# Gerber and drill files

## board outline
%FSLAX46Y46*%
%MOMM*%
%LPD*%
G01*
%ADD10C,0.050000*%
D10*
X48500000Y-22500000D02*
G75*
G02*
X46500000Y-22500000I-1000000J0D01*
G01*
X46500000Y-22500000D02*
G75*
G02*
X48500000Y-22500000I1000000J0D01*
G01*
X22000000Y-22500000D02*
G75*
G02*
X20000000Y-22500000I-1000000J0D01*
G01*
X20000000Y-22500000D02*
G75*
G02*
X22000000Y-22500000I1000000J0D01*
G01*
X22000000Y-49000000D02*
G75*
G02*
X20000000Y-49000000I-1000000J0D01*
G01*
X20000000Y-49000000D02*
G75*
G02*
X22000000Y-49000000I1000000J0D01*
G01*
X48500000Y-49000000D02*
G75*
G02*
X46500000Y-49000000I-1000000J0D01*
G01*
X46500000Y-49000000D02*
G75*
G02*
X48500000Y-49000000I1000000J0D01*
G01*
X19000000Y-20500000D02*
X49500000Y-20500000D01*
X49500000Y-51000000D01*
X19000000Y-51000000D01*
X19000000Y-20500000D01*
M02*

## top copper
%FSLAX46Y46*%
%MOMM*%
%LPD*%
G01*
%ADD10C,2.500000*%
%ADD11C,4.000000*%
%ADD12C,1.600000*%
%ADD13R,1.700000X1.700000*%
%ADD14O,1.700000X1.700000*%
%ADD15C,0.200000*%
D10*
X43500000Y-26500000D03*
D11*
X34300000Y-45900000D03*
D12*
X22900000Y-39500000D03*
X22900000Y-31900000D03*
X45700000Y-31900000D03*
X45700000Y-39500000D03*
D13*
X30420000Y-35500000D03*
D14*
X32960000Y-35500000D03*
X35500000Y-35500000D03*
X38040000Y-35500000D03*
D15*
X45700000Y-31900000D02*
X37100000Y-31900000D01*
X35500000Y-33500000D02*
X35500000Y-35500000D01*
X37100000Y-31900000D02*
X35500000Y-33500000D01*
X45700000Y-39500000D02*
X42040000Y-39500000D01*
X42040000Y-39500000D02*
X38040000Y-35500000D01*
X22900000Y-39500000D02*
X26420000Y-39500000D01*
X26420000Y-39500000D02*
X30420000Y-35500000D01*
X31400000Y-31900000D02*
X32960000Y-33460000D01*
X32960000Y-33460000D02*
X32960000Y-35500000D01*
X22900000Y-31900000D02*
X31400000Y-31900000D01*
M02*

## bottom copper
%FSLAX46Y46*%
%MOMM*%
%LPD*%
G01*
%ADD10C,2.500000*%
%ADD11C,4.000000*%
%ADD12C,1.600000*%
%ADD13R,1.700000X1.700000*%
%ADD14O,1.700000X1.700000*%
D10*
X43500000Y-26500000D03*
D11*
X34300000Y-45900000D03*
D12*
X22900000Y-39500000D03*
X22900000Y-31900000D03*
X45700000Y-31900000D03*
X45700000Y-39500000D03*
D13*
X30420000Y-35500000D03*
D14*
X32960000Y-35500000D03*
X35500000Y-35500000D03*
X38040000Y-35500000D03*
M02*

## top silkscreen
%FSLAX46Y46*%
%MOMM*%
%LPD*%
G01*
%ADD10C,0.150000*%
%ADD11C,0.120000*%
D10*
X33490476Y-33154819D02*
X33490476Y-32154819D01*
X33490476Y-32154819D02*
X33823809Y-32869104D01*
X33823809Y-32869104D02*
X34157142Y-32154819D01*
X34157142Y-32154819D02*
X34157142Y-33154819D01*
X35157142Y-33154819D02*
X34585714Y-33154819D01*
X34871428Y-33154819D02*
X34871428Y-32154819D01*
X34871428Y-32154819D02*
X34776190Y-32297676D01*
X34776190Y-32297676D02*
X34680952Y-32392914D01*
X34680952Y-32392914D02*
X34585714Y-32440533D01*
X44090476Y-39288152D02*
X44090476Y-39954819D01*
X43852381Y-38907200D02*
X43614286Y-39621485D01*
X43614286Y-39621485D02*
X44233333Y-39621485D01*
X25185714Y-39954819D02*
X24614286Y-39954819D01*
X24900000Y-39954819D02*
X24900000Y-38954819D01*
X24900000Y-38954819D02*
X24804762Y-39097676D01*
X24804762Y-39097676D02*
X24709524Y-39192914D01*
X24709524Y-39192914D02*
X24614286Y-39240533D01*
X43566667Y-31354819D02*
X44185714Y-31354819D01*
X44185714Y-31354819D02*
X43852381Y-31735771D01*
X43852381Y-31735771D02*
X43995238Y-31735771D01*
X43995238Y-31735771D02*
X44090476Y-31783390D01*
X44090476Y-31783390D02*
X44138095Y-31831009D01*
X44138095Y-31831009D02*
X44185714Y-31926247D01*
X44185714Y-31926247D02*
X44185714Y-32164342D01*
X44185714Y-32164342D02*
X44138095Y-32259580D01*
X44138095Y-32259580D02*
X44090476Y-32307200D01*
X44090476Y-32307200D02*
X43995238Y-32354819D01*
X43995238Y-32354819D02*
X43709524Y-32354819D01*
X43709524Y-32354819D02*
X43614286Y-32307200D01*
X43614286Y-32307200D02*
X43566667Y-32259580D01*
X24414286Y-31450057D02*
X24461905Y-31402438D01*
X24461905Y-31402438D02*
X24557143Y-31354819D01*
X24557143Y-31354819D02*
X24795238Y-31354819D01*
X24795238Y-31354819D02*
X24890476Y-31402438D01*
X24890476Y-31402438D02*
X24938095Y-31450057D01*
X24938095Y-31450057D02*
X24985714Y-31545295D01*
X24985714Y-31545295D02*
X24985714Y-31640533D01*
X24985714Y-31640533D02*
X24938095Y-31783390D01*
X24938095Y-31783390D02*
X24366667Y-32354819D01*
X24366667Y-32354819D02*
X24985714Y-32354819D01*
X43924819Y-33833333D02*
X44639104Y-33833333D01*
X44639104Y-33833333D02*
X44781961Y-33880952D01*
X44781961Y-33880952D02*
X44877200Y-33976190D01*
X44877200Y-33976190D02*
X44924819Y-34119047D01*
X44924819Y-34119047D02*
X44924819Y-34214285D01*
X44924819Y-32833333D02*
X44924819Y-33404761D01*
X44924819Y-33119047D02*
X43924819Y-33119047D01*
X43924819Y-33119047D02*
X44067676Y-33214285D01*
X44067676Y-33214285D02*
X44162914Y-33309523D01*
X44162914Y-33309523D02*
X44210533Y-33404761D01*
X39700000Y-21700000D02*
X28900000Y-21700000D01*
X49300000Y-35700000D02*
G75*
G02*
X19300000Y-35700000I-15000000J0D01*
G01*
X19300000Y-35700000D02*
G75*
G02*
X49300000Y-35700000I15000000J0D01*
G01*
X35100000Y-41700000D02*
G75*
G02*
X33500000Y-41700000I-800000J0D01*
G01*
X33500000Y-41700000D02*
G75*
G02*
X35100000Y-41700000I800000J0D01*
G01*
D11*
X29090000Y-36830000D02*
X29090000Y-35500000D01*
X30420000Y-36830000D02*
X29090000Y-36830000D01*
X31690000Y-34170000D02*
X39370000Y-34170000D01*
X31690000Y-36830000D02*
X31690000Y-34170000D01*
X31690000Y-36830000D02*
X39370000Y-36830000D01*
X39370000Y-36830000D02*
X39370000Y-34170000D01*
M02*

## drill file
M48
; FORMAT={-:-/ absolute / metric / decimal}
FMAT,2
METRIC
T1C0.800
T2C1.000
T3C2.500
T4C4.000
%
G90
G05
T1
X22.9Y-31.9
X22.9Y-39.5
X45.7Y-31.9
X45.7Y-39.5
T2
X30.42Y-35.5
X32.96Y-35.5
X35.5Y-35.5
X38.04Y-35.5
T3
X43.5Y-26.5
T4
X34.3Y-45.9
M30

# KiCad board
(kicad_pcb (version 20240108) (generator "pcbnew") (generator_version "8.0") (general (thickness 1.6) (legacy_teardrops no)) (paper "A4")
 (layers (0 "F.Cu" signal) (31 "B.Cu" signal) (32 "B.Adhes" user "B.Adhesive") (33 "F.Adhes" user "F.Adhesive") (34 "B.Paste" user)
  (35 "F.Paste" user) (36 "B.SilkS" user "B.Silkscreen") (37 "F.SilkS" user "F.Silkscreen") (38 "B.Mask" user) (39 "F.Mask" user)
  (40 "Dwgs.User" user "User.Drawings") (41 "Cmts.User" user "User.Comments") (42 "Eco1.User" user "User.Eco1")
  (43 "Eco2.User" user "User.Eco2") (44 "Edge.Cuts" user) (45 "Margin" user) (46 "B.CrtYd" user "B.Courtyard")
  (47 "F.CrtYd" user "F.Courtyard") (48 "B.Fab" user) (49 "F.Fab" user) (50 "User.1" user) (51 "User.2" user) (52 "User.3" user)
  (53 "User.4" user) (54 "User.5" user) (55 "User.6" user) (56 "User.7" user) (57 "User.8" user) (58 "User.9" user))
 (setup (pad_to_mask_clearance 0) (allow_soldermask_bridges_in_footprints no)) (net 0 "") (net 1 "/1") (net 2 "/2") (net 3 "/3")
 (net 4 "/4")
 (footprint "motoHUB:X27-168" (layer "F.Cu") (at 34.3 35.7 180)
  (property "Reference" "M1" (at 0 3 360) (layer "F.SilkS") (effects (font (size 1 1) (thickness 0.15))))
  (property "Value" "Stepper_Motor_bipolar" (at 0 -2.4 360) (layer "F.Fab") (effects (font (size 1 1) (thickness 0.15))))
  (fp_line (start -5.4 14) (end 5.4 14) (stroke (width 0.15) (type solid)) (layer "F.SilkS"))
  (fp_circle (center 0 0) (end 15 0) (stroke (width 0.15) (type solid)) (fill none) (layer "F.SilkS"))
  (fp_circle (center 0 -6) (end 0.8 -6) (stroke (width 0.15) (type solid)) (fill none) (layer "F.SilkS"))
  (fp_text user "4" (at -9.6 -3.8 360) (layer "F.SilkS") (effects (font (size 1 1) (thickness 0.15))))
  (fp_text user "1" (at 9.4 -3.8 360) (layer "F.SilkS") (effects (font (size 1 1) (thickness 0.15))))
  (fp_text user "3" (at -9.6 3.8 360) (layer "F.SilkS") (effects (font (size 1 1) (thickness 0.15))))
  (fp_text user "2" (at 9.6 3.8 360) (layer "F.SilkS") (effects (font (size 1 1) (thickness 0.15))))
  (pad "" thru_hole circle (at -9.2 9.2 180) (size 2.5 2.5) (drill 2.5) (layers "*.Cu" "*.Mask") (remove_unused_layers no))
  (pad "" thru_hole circle (at 0 -10.2 180) (size 4 4) (drill 4) (layers "*.Cu" "*.Mask") (remove_unused_layers no))
  (pad "1" thru_hole circle (at 11.4 -3.8 180) (size 1.6 1.6) (drill 0.8) (layers "*.Cu" "*.Mask") (remove_unused_layers no) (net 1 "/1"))
  (pad "2" thru_hole circle (at 11.4 3.8 180) (size 1.6 1.6) (drill 0.8) (layers "*.Cu" "*.Mask") (remove_unused_layers no) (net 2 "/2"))
  (pad "3" thru_hole circle (at -11.4 3.8 180) (size 1.6 1.6) (drill 0.8) (layers "*.Cu" "*.Mask") (remove_unused_layers no) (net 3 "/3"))
  (pad "4" thru_hole circle (at -11.4 -3.8 180) (size 1.6 1.6) (drill 0.8) (layers "*.Cu" "*.Mask") (remove_unused_layers no) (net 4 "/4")))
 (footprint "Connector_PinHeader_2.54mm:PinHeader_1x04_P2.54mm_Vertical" (layer "F.Cu") (at 30.42 35.5 90)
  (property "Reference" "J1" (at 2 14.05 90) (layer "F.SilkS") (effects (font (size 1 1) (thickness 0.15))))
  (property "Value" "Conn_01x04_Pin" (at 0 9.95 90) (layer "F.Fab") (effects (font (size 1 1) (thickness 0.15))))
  (fp_line (start -1.33 -1.33) (end 0 -1.33) (stroke (width 0.12) (type solid)) (layer "F.SilkS"))
  (fp_line (start -1.33 0) (end -1.33 -1.33) (stroke (width 0.12) (type solid)) (layer "F.SilkS"))
  (fp_line (start 1.33 1.27) (end 1.33 8.95) (stroke (width 0.12) (type solid)) (layer "F.SilkS"))
  (fp_line (start -1.33 1.27) (end 1.33 1.27) (stroke (width 0.12) (type solid)) (layer "F.SilkS"))
  (fp_line (start -1.33 1.27) (end -1.33 8.95) (stroke (width 0.12) (type solid)) (layer "F.SilkS"))
  (fp_line (start -1.33 8.95) (end 1.33 8.95) (stroke (width 0.12) (type solid)) (layer "F.SilkS"))
  (pad "1" thru_hole rect (at 0 0 90) (size 1.7 1.7) (drill 1) (layers "*.Cu" "*.Mask") (remove_unused_layers no) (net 1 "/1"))
  (pad "2" thru_hole oval (at 0 2.54 90) (size 1.7 1.7) (drill 1) (layers "*.Cu" "*.Mask") (remove_unused_layers no) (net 2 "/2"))
  (pad "3" thru_hole oval (at 0 5.08 90) (size 1.7 1.7) (drill 1) (layers "*.Cu" "*.Mask") (remove_unused_layers no) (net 3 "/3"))
  (pad "4" thru_hole oval (at 0 7.62 90) (size 1.7 1.7) (drill 1) (layers "*.Cu" "*.Mask") (remove_unused_layers no) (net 4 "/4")))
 (gr_circle (center 47.5 22.5) (end 48.5 22.5) (stroke (width 0.05) (type default)) (fill none) (layer "Edge.Cuts"))
 (gr_circle (center 21 22.5) (end 22 22.5) (stroke (width 0.05) (type default)) (fill none) (layer "Edge.Cuts"))
 (gr_circle (center 21 49) (end 22 49) (stroke (width 0.05) (type default)) (fill none) (layer "Edge.Cuts"))
 (gr_circle (center 47.5 49) (end 48.5 49) (stroke (width 0.05) (type default)) (fill none) (layer "Edge.Cuts"))
 (gr_rect (start 19 20.5) (end 49.5 51) (stroke (width 0.05) (type default)) (fill none) (layer "Edge.Cuts"))
 (segment (start 45.7 31.9) (end 37.1 31.9) (width 0.2) (layer "F.Cu") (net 3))
 (segment (start 35.5 33.5) (end 35.5 35.5) (width 0.2) (layer "F.Cu") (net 3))
 (segment (start 37.1 31.9) (end 35.5 33.5) (width 0.2) (layer "F.Cu") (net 3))
 (segment (start 45.7 39.5) (end 42.04 39.5) (width 0.2) (layer "F.Cu") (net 4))
 (segment (start 42.04 39.5) (end 38.04 35.5) (width 0.2) (layer "F.Cu") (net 4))
 (segment (start 22.9 39.5) (end 26.42 39.5) (width 0.2) (layer "F.Cu") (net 1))
 (segment (start 26.42 39.5) (end 30.42 35.5) (width 0.2) (layer "F.Cu") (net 1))
 (segment (start 31.4 31.9) (end 32.96 33.46) (width 0.2) (layer "F.Cu") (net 2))
 (segment (start 32.96 33.46) (end 32.96 35.5) (width 0.2) (layer "F.Cu") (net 2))
 (segment (start 22.9 31.9) (end 31.4 31.9) (width 0.2) (layer "F.Cu") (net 2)))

